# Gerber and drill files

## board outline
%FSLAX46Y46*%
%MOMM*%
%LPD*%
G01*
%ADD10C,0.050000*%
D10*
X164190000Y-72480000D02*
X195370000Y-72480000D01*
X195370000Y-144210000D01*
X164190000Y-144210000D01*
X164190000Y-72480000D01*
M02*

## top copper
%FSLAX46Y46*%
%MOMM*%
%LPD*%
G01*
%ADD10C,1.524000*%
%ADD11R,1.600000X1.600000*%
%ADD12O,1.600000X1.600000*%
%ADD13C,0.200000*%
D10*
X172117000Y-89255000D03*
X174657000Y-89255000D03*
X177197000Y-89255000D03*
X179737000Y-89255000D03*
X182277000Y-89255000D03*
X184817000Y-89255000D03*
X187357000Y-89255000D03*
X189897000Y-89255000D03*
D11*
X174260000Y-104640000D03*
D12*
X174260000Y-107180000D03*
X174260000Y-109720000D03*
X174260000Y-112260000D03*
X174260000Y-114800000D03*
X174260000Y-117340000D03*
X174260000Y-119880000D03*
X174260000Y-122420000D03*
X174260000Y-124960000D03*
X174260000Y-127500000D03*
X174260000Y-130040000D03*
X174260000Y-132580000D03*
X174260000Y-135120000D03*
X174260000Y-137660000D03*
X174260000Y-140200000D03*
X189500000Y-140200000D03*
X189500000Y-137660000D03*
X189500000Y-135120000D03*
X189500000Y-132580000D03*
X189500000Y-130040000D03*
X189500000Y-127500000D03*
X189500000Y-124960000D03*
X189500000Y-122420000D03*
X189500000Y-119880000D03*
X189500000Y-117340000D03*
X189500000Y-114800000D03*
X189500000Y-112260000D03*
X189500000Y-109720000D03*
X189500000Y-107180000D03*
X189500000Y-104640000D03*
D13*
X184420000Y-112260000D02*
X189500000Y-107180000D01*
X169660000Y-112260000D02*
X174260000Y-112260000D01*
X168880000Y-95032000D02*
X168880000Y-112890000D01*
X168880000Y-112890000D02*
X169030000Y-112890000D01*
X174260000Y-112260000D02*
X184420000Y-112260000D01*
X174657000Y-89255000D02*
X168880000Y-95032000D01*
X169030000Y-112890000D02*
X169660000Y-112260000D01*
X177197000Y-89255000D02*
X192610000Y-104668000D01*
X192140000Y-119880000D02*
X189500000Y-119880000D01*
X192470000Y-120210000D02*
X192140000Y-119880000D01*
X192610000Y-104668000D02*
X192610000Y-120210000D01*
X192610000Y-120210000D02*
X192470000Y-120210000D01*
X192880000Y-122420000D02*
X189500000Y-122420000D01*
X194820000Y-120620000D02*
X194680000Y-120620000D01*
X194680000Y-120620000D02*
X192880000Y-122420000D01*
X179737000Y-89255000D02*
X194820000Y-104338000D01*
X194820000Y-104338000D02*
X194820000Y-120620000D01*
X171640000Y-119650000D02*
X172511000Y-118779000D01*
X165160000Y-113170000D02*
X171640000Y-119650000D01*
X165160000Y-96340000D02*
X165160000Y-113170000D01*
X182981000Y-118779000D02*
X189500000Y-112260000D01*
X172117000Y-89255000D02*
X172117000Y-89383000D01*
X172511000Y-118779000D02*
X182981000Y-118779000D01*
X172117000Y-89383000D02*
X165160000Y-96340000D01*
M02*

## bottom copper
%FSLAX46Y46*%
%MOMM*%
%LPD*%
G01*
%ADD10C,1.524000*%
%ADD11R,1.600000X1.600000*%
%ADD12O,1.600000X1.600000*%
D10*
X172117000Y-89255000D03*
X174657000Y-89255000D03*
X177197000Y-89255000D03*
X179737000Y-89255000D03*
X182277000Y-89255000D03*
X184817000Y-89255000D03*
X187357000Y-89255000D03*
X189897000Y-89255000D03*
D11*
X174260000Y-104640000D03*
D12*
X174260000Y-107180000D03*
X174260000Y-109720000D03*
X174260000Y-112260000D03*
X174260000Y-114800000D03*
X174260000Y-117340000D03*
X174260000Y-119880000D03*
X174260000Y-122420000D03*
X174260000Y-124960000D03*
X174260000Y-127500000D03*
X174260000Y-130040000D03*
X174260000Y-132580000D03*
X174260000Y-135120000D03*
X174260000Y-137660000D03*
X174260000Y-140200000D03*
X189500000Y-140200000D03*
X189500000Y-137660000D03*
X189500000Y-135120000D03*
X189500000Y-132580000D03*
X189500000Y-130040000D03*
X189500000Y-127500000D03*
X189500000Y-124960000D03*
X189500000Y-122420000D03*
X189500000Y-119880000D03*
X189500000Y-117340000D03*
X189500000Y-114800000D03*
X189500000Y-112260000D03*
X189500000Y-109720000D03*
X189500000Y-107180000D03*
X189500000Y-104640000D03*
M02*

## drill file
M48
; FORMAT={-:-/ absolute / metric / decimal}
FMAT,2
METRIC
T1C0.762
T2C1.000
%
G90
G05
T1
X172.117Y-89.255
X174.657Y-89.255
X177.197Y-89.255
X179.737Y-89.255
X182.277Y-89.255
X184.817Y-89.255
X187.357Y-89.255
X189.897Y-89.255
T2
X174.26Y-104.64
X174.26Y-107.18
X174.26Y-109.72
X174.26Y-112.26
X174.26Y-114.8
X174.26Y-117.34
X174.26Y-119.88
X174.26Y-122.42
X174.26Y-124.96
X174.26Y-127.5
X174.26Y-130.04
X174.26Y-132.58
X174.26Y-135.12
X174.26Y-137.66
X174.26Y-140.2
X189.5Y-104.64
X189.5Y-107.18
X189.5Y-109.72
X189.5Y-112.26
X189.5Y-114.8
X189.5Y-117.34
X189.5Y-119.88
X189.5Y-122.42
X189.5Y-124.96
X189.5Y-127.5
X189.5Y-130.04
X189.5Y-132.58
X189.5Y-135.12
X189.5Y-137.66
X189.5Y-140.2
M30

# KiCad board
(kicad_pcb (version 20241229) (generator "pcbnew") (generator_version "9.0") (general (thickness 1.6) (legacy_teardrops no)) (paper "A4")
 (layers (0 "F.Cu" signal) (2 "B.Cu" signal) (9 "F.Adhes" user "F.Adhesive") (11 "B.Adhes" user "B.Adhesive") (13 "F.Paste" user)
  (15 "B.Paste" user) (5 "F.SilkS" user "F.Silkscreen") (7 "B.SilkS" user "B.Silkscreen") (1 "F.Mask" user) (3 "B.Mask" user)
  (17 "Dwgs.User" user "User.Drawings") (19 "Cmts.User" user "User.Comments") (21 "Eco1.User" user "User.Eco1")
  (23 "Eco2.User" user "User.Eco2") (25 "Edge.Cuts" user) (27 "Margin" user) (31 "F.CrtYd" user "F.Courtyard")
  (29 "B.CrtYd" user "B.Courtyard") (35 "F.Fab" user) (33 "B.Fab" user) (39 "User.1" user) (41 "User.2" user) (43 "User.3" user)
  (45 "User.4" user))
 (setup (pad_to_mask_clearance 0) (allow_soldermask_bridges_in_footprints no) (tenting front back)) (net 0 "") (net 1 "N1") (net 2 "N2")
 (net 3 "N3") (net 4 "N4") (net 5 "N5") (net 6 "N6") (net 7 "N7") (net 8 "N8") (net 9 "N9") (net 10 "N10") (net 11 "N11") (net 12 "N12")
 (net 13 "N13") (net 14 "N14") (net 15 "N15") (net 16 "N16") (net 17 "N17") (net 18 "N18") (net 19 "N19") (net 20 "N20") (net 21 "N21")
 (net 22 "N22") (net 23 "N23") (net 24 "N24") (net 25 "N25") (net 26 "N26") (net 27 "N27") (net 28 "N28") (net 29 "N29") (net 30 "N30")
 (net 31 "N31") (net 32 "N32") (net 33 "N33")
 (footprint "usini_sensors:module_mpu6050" (layer "F.Cu") (at 189.897 89.255 90)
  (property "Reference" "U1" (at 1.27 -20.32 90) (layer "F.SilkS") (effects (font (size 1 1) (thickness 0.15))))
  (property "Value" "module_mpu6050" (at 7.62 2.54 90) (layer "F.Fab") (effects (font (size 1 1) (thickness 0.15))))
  (pad "1" thru_hole circle (at 0 -17.78 90) (size 1.524 1.524) (drill 0.762) (layers "*.Cu" "*.Mask") (remove_unused_layers no)
   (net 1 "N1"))
  (pad "2" thru_hole circle (at 0 -15.24 90) (size 1.524 1.524) (drill 0.762) (layers "*.Cu" "*.Mask") (remove_unused_layers no)
   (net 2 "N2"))
  (pad "3" thru_hole circle (at 0 -12.7 90) (size 1.524 1.524) (drill 0.762) (layers "*.Cu" "*.Mask") (remove_unused_layers no) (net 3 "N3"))
  (pad "4" thru_hole circle (at 0 -10.16 90) (size 1.524 1.524) (drill 0.762) (layers "*.Cu" "*.Mask") (remove_unused_layers no)
   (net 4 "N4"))
  (pad "5" thru_hole circle (at 0 -7.62 90) (size 1.524 1.524) (drill 0.762) (layers "*.Cu" "*.Mask") (remove_unused_layers no) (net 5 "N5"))
  (pad "6" thru_hole circle (at 0 -5.08 90) (size 1.524 1.524) (drill 0.762) (layers "*.Cu" "*.Mask") (remove_unused_layers no) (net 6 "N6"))
  (pad "7" thru_hole circle (at 0 -2.54 90) (size 1.524 1.524) (drill 0.762) (layers "*.Cu" "*.Mask") (remove_unused_layers no) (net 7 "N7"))
  (pad "8" thru_hole circle (at 0 0 90) (size 1.524 1.524) (drill 0.762) (layers "*.Cu" "*.Mask") (remove_unused_layers no) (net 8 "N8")))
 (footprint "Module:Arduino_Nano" (layer "F.Cu") (at 174.26 104.64)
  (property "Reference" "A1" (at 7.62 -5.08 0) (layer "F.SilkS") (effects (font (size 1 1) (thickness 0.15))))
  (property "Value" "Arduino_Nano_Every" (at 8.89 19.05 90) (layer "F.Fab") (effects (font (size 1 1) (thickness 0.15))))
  (pad "1" thru_hole rect (at 0 0) (size 1.6 1.6) (drill 1) (layers "*.Cu" "*.Mask") (remove_unused_layers no) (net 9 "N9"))
  (pad "2" thru_hole oval (at 0 2.54) (size 1.6 1.6) (drill 1) (layers "*.Cu" "*.Mask") (remove_unused_layers no) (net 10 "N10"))
  (pad "3" thru_hole oval (at 0 5.08) (size 1.6 1.6) (drill 1) (layers "*.Cu" "*.Mask") (remove_unused_layers no) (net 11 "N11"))
  (pad "4" thru_hole oval (at 0 7.62) (size 1.6 1.6) (drill 1) (layers "*.Cu" "*.Mask") (remove_unused_layers no) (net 2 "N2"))
  (pad "5" thru_hole oval (at 0 10.16) (size 1.6 1.6) (drill 1) (layers "*.Cu" "*.Mask") (remove_unused_layers no) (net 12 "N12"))
  (pad "6" thru_hole oval (at 0 12.7) (size 1.6 1.6) (drill 1) (layers "*.Cu" "*.Mask") (remove_unused_layers no) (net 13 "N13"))
  (pad "7" thru_hole oval (at 0 15.24) (size 1.6 1.6) (drill 1) (layers "*.Cu" "*.Mask") (remove_unused_layers no) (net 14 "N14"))
  (pad "8" thru_hole oval (at 0 17.78) (size 1.6 1.6) (drill 1) (layers "*.Cu" "*.Mask") (remove_unused_layers no) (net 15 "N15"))
  (pad "9" thru_hole oval (at 0 20.32) (size 1.6 1.6) (drill 1) (layers "*.Cu" "*.Mask") (remove_unused_layers no) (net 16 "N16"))
  (pad "10" thru_hole oval (at 0 22.86) (size 1.6 1.6) (drill 1) (layers "*.Cu" "*.Mask") (remove_unused_layers no) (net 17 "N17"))
  (pad "11" thru_hole oval (at 0 25.4) (size 1.6 1.6) (drill 1) (layers "*.Cu" "*.Mask") (remove_unused_layers no) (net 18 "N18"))
  (pad "12" thru_hole oval (at 0 27.94) (size 1.6 1.6) (drill 1) (layers "*.Cu" "*.Mask") (remove_unused_layers no) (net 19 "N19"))
  (pad "13" thru_hole oval (at 0 30.48) (size 1.6 1.6) (drill 1) (layers "*.Cu" "*.Mask") (remove_unused_layers no) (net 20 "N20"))
  (pad "14" thru_hole oval (at 0 33.02) (size 1.6 1.6) (drill 1) (layers "*.Cu" "*.Mask") (remove_unused_layers no) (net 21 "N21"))
  (pad "15" thru_hole oval (at 0 35.56) (size 1.6 1.6) (drill 1) (layers "*.Cu" "*.Mask") (remove_unused_layers no) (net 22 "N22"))
  (pad "16" thru_hole oval (at 15.24 35.56) (size 1.6 1.6) (drill 1) (layers "*.Cu" "*.Mask") (remove_unused_layers no) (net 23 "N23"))
  (pad "17" thru_hole oval (at 15.24 33.02) (size 1.6 1.6) (drill 1) (layers "*.Cu" "*.Mask") (remove_unused_layers no) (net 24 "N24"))
  (pad "18" thru_hole oval (at 15.24 30.48) (size 1.6 1.6) (drill 1) (layers "*.Cu" "*.Mask") (remove_unused_layers no) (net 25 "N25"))
  (pad "19" thru_hole oval (at 15.24 27.94) (size 1.6 1.6) (drill 1) (layers "*.Cu" "*.Mask") (remove_unused_layers no) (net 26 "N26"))
  (pad "20" thru_hole oval (at 15.24 25.4) (size 1.6 1.6) (drill 1) (layers "*.Cu" "*.Mask") (remove_unused_layers no) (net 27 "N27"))
  (pad "21" thru_hole oval (at 15.24 22.86) (size 1.6 1.6) (drill 1) (layers "*.Cu" "*.Mask") (remove_unused_layers no) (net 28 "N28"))
  (pad "22" thru_hole oval (at 15.24 20.32) (size 1.6 1.6) (drill 1) (layers "*.Cu" "*.Mask") (remove_unused_layers no) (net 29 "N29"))
  (pad "23" thru_hole oval (at 15.24 17.78) (size 1.6 1.6) (drill 1) (layers "*.Cu" "*.Mask") (remove_unused_layers no) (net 4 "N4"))
  (pad "24" thru_hole oval (at 15.24 15.24) (size 1.6 1.6) (drill 1) (layers "*.Cu" "*.Mask") (remove_unused_layers no) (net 3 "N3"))
  (pad "25" thru_hole oval (at 15.24 12.7) (size 1.6 1.6) (drill 1) (layers "*.Cu" "*.Mask") (remove_unused_layers no) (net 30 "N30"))
  (pad "26" thru_hole oval (at 15.24 10.16) (size 1.6 1.6) (drill 1) (layers "*.Cu" "*.Mask") (remove_unused_layers no) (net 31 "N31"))
  (pad "27" thru_hole oval (at 15.24 7.62) (size 1.6 1.6) (drill 1) (layers "*.Cu" "*.Mask") (remove_unused_layers no) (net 1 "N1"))
  (pad "28" thru_hole oval (at 15.24 5.08) (size 1.6 1.6) (drill 1) (layers "*.Cu" "*.Mask") (remove_unused_layers no) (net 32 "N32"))
  (pad "29" thru_hole oval (at 15.24 2.54) (size 1.6 1.6) (drill 1) (layers "*.Cu" "*.Mask") (remove_unused_layers no) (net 2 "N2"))
  (pad "30" thru_hole oval (at 15.24 0) (size 1.6 1.6) (drill 1) (layers "*.Cu" "*.Mask") (remove_unused_layers no) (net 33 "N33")))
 (gr_rect (start 164.19 72.48) (end 195.37 144.21) (stroke (width 0.05) (type default)) (fill no) (layer "Edge.Cuts"))
 (segment (start 184.42 112.26) (end 189.5 107.18) (width 0.2) (layer "F.Cu") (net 2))
 (segment (start 169.66 112.26) (end 174.26 112.26) (width 0.2) (layer "F.Cu") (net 2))
 (segment (start 168.88 95.032) (end 168.88 112.89) (width 0.2) (layer "F.Cu") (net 2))
 (segment (start 168.88 112.89) (end 169.03 112.89) (width 0.2) (layer "F.Cu") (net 2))
 (segment (start 174.26 112.26) (end 184.42 112.26) (width 0.2) (layer "F.Cu") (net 2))
 (segment (start 174.657 89.255) (end 168.88 95.032) (width 0.2) (layer "F.Cu") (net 2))
 (segment (start 169.03 112.89) (end 169.66 112.26) (width 0.2) (layer "F.Cu") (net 2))
 (segment (start 177.197 89.255) (end 192.61 104.668) (width 0.2) (layer "F.Cu") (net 3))
 (segment (start 192.14 119.88) (end 189.5 119.88) (width 0.2) (layer "F.Cu") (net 3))
 (segment (start 192.47 120.21) (end 192.14 119.88) (width 0.2) (layer "F.Cu") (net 3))
 (segment (start 192.61 104.668) (end 192.61 120.21) (width 0.2) (layer "F.Cu") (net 3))
 (segment (start 192.61 120.21) (end 192.47 120.21) (width 0.2) (layer "F.Cu") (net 3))
 (segment (start 192.88 122.42) (end 189.5 122.42) (width 0.2) (layer "F.Cu") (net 4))
 (segment (start 194.82 120.62) (end 194.68 120.62) (width 0.2) (layer "F.Cu") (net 4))
 (segment (start 194.68 120.62) (end 192.88 122.42) (width 0.2) (layer "F.Cu") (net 4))
 (segment (start 179.737 89.255) (end 194.82 104.338) (width 0.2) (layer "F.Cu") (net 4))
 (segment (start 194.82 104.338) (end 194.82 120.62) (width 0.2) (layer "F.Cu") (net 4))
 (segment (start 171.64 119.65) (end 172.511 118.779) (width 0.2) (layer "F.Cu") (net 1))
 (segment (start 165.16 113.17) (end 171.64 119.65) (width 0.2) (layer "F.Cu") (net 1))
 (segment (start 165.16 96.34) (end 165.16 113.17) (width 0.2) (layer "F.Cu") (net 1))
 (segment (start 182.981 118.779) (end 189.5 112.26) (width 0.2) (layer "F.Cu") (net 1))
 (segment (start 172.117 89.255) (end 172.117 89.383) (width 0.2) (layer "F.Cu") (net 1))
 (segment (start 172.511 118.779) (end 182.981 118.779) (width 0.2) (layer "F.Cu") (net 1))
 (segment (start 172.117 89.383) (end 165.16 96.34) (width 0.2) (layer "F.Cu") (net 1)))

